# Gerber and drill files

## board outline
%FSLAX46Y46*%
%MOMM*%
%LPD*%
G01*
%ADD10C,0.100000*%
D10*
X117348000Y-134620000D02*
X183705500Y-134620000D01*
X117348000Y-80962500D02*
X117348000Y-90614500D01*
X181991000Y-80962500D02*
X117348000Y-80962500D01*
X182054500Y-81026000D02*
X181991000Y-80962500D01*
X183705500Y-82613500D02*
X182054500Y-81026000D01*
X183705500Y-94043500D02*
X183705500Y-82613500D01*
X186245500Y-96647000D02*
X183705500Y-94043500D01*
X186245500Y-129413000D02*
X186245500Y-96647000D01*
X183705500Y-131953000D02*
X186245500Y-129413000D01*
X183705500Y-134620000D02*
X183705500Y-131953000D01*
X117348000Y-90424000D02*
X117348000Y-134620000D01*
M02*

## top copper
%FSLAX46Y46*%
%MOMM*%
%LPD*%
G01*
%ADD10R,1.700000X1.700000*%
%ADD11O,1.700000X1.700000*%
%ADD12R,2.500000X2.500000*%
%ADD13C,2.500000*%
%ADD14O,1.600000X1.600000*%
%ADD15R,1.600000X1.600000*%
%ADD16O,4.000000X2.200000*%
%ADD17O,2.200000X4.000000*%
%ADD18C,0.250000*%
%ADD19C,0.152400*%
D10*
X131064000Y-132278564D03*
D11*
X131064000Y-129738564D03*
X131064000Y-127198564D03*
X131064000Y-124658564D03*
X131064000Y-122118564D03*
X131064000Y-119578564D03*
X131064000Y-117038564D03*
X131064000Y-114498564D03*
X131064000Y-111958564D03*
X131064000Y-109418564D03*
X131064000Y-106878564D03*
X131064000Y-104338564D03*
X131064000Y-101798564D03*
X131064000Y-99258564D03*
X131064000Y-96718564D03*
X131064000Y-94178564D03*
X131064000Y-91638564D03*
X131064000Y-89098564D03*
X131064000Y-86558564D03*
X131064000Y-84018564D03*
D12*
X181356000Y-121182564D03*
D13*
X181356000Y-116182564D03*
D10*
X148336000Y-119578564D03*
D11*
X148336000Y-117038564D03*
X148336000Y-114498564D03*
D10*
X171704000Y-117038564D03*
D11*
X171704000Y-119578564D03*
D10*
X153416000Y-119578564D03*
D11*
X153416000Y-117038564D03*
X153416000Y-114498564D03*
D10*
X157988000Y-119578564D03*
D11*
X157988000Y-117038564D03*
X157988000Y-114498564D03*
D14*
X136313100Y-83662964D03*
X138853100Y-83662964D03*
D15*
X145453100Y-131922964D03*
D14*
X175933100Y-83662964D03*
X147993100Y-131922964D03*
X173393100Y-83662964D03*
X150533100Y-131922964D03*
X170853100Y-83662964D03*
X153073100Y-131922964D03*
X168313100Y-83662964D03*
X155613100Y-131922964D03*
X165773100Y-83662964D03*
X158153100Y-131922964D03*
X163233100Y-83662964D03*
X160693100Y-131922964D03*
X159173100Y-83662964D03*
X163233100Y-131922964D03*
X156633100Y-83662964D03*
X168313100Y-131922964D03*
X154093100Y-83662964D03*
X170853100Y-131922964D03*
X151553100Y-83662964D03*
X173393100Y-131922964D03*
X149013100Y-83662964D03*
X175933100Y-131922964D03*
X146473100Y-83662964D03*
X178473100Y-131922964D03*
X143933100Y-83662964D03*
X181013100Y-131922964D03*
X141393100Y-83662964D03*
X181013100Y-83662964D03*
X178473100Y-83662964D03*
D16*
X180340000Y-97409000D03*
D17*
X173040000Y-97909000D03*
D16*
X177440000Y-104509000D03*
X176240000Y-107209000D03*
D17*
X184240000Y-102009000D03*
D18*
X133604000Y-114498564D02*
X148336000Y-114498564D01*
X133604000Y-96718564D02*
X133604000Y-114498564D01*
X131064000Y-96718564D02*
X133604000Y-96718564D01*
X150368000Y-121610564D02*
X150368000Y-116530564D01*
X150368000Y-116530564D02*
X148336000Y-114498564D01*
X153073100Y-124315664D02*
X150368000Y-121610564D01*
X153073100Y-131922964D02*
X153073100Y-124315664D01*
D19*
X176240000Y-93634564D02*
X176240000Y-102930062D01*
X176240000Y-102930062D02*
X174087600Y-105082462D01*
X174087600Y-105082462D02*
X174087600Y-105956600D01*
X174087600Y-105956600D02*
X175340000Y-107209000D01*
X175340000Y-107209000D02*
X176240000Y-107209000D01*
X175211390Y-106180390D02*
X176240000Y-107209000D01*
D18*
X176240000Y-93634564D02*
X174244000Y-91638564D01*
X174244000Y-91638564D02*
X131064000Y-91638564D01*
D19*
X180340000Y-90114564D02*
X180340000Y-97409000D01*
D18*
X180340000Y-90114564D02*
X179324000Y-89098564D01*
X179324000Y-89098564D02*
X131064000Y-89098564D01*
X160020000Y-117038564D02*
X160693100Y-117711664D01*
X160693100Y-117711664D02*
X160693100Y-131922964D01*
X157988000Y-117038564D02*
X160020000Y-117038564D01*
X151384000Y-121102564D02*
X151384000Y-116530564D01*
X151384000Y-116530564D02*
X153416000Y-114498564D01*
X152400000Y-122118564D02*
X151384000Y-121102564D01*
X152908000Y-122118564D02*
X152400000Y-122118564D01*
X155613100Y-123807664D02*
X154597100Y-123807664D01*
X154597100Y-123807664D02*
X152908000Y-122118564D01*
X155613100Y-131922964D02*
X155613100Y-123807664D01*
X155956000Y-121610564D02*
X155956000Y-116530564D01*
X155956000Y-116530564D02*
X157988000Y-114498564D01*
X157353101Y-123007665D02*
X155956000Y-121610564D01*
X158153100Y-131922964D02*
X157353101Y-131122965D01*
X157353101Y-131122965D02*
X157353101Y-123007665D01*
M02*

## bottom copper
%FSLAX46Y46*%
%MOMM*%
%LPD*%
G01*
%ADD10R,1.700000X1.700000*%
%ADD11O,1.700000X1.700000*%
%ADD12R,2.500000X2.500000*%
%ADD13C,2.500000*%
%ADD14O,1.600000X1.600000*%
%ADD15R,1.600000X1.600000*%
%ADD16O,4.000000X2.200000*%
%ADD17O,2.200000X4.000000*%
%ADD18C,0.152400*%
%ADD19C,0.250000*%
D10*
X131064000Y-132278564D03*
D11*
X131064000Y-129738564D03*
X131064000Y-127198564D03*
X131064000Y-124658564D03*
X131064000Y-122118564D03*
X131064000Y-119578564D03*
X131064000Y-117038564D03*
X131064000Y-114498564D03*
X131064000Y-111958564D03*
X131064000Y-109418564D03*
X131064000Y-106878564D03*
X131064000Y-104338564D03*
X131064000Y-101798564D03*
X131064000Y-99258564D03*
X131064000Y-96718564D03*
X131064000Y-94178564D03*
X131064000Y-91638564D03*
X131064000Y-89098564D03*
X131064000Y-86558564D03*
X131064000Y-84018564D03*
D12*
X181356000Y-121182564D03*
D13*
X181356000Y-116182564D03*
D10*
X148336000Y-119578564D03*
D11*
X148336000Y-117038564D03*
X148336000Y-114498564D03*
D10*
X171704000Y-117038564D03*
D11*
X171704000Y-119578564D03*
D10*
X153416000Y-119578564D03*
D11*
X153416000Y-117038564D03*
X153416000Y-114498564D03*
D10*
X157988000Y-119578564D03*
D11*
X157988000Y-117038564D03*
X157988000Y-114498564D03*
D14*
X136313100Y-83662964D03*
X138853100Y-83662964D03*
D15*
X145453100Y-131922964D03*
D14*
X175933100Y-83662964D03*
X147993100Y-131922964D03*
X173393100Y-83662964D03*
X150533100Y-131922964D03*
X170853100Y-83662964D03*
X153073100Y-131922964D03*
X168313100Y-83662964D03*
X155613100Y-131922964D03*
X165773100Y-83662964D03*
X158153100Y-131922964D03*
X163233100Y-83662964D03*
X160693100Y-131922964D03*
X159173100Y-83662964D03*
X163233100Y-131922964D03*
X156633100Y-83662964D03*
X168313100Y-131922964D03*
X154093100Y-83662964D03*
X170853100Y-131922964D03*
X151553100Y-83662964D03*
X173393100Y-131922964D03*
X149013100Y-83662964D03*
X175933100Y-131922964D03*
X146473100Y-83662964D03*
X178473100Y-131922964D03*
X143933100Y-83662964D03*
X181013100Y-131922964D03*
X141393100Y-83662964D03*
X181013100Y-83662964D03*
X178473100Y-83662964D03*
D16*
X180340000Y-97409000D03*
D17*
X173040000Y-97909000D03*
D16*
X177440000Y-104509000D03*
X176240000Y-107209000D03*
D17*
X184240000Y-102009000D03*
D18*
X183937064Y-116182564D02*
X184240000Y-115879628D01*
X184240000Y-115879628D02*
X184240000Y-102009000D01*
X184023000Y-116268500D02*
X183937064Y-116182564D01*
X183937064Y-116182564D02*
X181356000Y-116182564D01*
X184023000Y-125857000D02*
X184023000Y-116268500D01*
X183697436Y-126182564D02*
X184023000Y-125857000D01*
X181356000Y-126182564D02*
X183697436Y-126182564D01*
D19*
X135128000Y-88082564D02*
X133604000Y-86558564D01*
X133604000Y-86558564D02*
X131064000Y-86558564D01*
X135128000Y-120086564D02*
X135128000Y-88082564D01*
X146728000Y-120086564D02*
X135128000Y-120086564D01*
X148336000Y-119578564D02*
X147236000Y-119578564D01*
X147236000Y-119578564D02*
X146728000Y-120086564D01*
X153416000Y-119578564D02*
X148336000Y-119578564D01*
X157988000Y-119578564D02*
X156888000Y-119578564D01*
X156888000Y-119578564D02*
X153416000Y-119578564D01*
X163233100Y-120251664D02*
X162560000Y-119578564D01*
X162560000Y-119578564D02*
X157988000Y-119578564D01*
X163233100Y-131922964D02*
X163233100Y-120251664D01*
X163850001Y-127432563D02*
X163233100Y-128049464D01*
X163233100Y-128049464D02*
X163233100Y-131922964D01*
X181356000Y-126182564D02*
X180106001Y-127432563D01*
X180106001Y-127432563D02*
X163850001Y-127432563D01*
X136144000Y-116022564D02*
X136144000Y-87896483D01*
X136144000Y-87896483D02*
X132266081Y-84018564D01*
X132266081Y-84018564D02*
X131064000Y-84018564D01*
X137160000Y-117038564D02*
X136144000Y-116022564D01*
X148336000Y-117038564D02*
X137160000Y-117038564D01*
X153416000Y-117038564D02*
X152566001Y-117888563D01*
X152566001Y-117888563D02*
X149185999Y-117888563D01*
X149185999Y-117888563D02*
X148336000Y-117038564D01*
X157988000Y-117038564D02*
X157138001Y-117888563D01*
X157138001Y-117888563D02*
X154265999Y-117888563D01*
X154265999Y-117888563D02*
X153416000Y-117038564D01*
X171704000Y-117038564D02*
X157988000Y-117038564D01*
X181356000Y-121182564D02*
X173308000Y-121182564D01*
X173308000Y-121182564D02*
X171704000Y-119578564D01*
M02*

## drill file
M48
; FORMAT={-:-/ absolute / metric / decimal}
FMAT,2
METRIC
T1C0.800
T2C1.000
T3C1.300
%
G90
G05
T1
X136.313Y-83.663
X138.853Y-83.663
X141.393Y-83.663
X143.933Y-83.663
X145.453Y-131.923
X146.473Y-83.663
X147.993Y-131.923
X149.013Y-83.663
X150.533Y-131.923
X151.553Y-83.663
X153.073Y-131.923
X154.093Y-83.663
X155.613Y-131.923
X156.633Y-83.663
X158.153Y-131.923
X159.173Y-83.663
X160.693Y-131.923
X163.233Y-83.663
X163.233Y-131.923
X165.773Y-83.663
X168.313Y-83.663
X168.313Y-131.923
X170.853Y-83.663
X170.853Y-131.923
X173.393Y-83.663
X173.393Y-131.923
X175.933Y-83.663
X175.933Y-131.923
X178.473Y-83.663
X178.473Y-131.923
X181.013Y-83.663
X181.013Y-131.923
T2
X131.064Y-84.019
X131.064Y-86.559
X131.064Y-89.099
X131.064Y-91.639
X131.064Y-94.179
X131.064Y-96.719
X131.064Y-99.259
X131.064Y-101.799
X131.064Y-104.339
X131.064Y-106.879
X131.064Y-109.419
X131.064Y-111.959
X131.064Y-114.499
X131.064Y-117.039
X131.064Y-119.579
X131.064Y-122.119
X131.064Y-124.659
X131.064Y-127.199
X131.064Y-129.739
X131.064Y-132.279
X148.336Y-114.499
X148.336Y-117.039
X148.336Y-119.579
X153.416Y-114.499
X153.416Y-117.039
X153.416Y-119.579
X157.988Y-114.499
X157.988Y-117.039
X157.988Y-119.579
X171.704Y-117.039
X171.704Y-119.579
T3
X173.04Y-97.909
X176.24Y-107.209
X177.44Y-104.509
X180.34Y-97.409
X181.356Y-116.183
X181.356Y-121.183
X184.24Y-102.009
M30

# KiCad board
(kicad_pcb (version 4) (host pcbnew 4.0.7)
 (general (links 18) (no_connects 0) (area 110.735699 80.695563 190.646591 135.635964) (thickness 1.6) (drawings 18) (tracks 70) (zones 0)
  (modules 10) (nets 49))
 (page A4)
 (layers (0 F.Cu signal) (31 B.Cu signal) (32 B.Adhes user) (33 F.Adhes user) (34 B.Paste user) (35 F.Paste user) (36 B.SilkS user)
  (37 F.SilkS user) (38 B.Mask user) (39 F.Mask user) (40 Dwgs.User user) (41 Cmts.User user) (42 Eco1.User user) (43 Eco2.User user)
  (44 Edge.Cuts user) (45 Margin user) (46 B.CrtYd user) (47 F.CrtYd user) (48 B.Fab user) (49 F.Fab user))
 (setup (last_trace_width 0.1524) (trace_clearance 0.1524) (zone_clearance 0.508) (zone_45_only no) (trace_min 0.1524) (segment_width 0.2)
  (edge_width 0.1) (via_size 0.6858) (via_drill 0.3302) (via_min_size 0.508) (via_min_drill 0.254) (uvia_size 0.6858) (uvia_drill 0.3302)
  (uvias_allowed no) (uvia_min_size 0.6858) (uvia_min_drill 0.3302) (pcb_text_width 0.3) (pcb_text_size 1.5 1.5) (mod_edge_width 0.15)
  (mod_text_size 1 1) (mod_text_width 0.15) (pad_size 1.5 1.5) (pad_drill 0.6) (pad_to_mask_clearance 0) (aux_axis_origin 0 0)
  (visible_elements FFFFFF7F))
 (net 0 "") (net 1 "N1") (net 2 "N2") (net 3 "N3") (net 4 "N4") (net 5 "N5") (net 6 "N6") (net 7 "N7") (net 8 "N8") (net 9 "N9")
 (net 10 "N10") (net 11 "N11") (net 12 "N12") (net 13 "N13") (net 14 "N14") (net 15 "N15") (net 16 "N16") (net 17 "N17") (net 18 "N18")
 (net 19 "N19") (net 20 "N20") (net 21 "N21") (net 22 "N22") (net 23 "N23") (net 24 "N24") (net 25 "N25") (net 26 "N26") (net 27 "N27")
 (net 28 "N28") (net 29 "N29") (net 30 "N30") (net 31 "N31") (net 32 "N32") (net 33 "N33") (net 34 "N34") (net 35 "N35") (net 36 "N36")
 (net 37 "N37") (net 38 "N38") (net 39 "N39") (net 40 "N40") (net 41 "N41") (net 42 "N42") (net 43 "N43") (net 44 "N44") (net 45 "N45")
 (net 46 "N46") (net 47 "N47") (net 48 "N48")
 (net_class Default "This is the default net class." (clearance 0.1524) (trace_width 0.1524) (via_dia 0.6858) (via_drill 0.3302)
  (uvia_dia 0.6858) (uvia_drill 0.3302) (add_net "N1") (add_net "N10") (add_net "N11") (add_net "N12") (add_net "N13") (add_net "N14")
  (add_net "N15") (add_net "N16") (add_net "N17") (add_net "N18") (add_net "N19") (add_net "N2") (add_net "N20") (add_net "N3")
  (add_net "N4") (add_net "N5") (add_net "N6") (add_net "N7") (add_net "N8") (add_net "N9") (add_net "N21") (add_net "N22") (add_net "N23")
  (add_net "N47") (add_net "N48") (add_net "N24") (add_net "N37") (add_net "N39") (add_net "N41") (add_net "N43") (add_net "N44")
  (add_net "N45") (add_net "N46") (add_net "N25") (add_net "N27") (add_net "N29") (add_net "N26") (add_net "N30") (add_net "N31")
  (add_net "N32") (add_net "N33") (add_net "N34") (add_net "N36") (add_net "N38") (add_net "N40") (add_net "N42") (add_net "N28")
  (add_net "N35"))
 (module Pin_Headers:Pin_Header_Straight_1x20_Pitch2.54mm (layer B.Cu) (at 131.064 132.278564)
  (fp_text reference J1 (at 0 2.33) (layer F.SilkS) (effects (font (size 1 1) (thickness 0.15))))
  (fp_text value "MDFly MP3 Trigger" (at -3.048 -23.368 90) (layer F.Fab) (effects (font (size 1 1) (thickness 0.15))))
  (pad 1 thru_hole rect (at 0 0) (size 1.7 1.7) (drill 1) (layers *.Cu *.Mask) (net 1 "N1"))
  (pad 2 thru_hole oval (at 0 -2.54) (size 1.7 1.7) (drill 1) (layers *.Cu *.Mask) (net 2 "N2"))
  (pad 3 thru_hole oval (at 0 -5.08) (size 1.7 1.7) (drill 1) (layers *.Cu *.Mask) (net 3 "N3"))
  (pad 4 thru_hole oval (at 0 -7.62) (size 1.7 1.7) (drill 1) (layers *.Cu *.Mask) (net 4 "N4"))
  (pad 5 thru_hole oval (at 0 -10.16) (size 1.7 1.7) (drill 1) (layers *.Cu *.Mask) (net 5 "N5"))
  (pad 6 thru_hole oval (at 0 -12.7) (size 1.7 1.7) (drill 1) (layers *.Cu *.Mask) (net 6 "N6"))
  (pad 7 thru_hole oval (at 0 -15.24) (size 1.7 1.7) (drill 1) (layers *.Cu *.Mask) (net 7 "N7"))
  (pad 8 thru_hole oval (at 0 -17.78) (size 1.7 1.7) (drill 1) (layers *.Cu *.Mask) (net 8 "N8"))
  (pad 9 thru_hole oval (at 0 -20.32) (size 1.7 1.7) (drill 1) (layers *.Cu *.Mask) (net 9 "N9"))
  (pad 10 thru_hole oval (at 0 -22.86) (size 1.7 1.7) (drill 1) (layers *.Cu *.Mask) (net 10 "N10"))
  (pad 11 thru_hole oval (at 0 -25.4) (size 1.7 1.7) (drill 1) (layers *.Cu *.Mask) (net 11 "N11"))
  (pad 12 thru_hole oval (at 0 -27.94) (size 1.7 1.7) (drill 1) (layers *.Cu *.Mask) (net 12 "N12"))
  (pad 13 thru_hole oval (at 0 -30.48) (size 1.7 1.7) (drill 1) (layers *.Cu *.Mask) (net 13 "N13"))
  (pad 14 thru_hole oval (at 0 -33.02) (size 1.7 1.7) (drill 1) (layers *.Cu *.Mask) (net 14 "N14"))
  (pad 15 thru_hole oval (at 0 -35.56) (size 1.7 1.7) (drill 1) (layers *.Cu *.Mask) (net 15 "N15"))
  (pad 16 thru_hole oval (at 0 -38.1) (size 1.7 1.7) (drill 1) (layers *.Cu *.Mask) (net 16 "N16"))
  (pad 17 thru_hole oval (at 0 -40.64) (size 1.7 1.7) (drill 1) (layers *.Cu *.Mask) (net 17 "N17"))
  (pad 18 thru_hole oval (at 0 -43.18) (size 1.7 1.7) (drill 1) (layers *.Cu *.Mask) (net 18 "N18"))
  (pad 19 thru_hole oval (at 0 -45.72) (size 1.7 1.7) (drill 1) (layers *.Cu *.Mask) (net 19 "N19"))
  (pad 20 thru_hole oval (at 0 -48.26) (size 1.7 1.7) (drill 1) (layers *.Cu *.Mask) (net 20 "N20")))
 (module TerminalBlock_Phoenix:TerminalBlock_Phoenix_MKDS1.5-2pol (layer F.Cu) (at 181.356 121.182564 90)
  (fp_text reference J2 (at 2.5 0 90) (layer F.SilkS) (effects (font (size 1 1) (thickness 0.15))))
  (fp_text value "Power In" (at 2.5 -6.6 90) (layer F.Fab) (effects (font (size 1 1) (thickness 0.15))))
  (pad 1 thru_hole rect (at 0 0 90) (size 2.5 2.5) (drill 1.3) (layers *.Cu *.Mask) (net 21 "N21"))
  (pad 2 thru_hole circle (at 5 0 90) (size 2.5 2.5) (drill 1.3) (layers *.Cu *.Mask) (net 19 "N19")))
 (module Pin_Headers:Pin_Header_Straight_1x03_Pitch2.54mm (layer F.Cu) (at 148.336 119.578564 180)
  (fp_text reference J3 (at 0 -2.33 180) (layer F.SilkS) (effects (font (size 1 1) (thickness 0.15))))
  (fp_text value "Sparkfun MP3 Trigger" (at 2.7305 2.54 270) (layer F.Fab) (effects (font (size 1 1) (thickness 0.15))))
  (pad 1 thru_hole rect (at 0 0 180) (size 1.7 1.7) (drill 1) (layers *.Cu *.Mask) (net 19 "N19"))
  (pad 2 thru_hole oval (at 0 2.54 180) (size 1.7 1.7) (drill 1) (layers *.Cu *.Mask) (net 20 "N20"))
  (pad 3 thru_hole oval (at 0 5.08 180) (size 1.7 1.7) (drill 1) (layers *.Cu *.Mask) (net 15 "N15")))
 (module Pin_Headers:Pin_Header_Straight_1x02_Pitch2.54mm (layer F.Cu) (at 171.704 117.038564)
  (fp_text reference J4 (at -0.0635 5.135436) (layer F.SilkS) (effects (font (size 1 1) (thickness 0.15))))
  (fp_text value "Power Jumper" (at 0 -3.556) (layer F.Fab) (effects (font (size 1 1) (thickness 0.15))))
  (pad 1 thru_hole rect (at 0 0) (size 1.7 1.7) (drill 1) (layers *.Cu *.Mask) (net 20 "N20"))
  (pad 2 thru_hole oval (at 0 2.54) (size 1.7 1.7) (drill 1) (layers *.Cu *.Mask) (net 21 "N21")))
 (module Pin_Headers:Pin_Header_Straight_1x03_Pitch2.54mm (layer F.Cu) (at 153.416 119.578564 180)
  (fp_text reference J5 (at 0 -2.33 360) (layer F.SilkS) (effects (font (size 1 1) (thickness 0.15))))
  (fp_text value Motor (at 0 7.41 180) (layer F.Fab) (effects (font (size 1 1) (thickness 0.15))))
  (pad 1 thru_hole rect (at 0 0 180) (size 1.7 1.7) (drill 1) (layers *.Cu *.Mask) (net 19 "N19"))
  (pad 2 thru_hole oval (at 0 2.54 180) (size 1.7 1.7) (drill 1) (layers *.Cu *.Mask) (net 20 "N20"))
  (pad 3 thru_hole oval (at 0 5.08 180) (size 1.7 1.7) (drill 1) (layers *.Cu *.Mask) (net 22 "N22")))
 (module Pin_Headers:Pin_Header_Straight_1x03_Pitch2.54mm (layer F.Cu) (at 157.988 119.578564 180)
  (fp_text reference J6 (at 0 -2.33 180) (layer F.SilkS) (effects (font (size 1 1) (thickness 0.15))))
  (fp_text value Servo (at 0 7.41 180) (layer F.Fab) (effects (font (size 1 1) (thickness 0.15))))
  (pad 1 thru_hole rect (at 0 0 180) (size 1.7 1.7) (drill 1) (layers *.Cu *.Mask) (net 19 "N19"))
  (pad 2 thru_hole oval (at 0 2.54 180) (size 1.7 1.7) (drill 1) (layers *.Cu *.Mask) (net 20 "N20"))
  (pad 3 thru_hole oval (at 0 5.08 180) (size 1.7 1.7) (drill 1) (layers *.Cu *.Mask) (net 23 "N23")))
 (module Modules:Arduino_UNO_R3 (layer B.Cu) (at 145.4531 131.922964)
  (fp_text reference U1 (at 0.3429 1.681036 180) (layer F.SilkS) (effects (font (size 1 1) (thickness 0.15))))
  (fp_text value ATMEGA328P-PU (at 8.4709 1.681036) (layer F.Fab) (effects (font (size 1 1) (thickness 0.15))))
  (pad 32 thru_hole oval (at -9.14 -48.26 270) (size 1.6 1.6) (drill 0.8) (layers *.Cu *.Mask))
  (pad 31 thru_hole oval (at -6.6 -48.26 270) (size 1.6 1.6) (drill 0.8) (layers *.Cu *.Mask))
  (pad 1 thru_hole rect (at 0 0 270) (size 1.6 1.6) (drill 0.8) (layers *.Cu *.Mask) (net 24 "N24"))
  (pad 17 thru_hole oval (at 30.48 -48.26 270) (size 1.6 1.6) (drill 0.8) (layers *.Cu *.Mask) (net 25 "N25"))
  (pad 2 thru_hole oval (at 2.54 0 270) (size 1.6 1.6) (drill 0.8) (layers *.Cu *.Mask) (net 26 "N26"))
  (pad 18 thru_hole oval (at 27.94 -48.26 270) (size 1.6 1.6) (drill 0.8) (layers *.Cu *.Mask) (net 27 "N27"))
  (pad 3 thru_hole oval (at 5.08 0 270) (size 1.6 1.6) (drill 0.8) (layers *.Cu *.Mask) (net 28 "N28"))
  (pad 19 thru_hole oval (at 25.4 -48.26 270) (size 1.6 1.6) (drill 0.8) (layers *.Cu *.Mask) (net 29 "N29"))
  (pad 4 thru_hole oval (at 7.62 0 270) (size 1.6 1.6) (drill 0.8) (layers *.Cu *.Mask) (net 15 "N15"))
  (pad 20 thru_hole oval (at 22.86 -48.26 270) (size 1.6 1.6) (drill 0.8) (layers *.Cu *.Mask) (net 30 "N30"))
  (pad 5 thru_hole oval (at 10.16 0 270) (size 1.6 1.6) (drill 0.8) (layers *.Cu *.Mask) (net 22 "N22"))
  (pad 21 thru_hole oval (at 20.32 -48.26 270) (size 1.6 1.6) (drill 0.8) (layers *.Cu *.Mask) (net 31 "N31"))
  (pad 6 thru_hole oval (at 12.7 0 270) (size 1.6 1.6) (drill 0.8) (layers *.Cu *.Mask) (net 23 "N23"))
  (pad 22 thru_hole oval (at 17.78 -48.26 270) (size 1.6 1.6) (drill 0.8) (layers *.Cu *.Mask) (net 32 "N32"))
  (pad 7 thru_hole oval (at 15.24 0 270) (size 1.6 1.6) (drill 0.8) (layers *.Cu *.Mask) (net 20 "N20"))
  (pad 23 thru_hole oval (at 13.72 -48.26 270) (size 1.6 1.6) (drill 0.8) (layers *.Cu *.Mask) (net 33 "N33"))
  (pad 8 thru_hole oval (at 17.78 0 270) (size 1.6 1.6) (drill 0.8) (layers *.Cu *.Mask) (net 19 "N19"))
  (pad 24 thru_hole oval (at 11.18 -48.26 270) (size 1.6 1.6) (drill 0.8) (layers *.Cu *.Mask) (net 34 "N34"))
  (pad 9 thru_hole oval (at 22.86 0 270) (size 1.6 1.6) (drill 0.8) (layers *.Cu *.Mask) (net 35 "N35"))
  (pad 25 thru_hole oval (at 8.64 -48.26 270) (size 1.6 1.6) (drill 0.8) (layers *.Cu *.Mask) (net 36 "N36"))
  (pad 10 thru_hole oval (at 25.4 0 270) (size 1.6 1.6) (drill 0.8) (layers *.Cu *.Mask) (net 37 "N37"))
  (pad 26 thru_hole oval (at 6.1 -48.26 270) (size 1.6 1.6) (drill 0.8) (layers *.Cu *.Mask) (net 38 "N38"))
  (pad 11 thru_hole oval (at 27.94 0 270) (size 1.6 1.6) (drill 0.8) (layers *.Cu *.Mask) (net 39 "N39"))
  (pad 27 thru_hole oval (at 3.56 -48.26 270) (size 1.6 1.6) (drill 0.8) (layers *.Cu *.Mask) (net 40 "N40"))
  (pad 12 thru_hole oval (at 30.48 0 270) (size 1.6 1.6) (drill 0.8) (layers *.Cu *.Mask) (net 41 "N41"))
  (pad 28 thru_hole oval (at 1.02 -48.26 270) (size 1.6 1.6) (drill 0.8) (layers *.Cu *.Mask) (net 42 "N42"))
  (pad 13 thru_hole oval (at 33.02 0 270) (size 1.6 1.6) (drill 0.8) (layers *.Cu *.Mask) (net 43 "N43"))
  (pad 29 thru_hole oval (at -1.52 -48.26 270) (size 1.6 1.6) (drill 0.8) (layers *.Cu *.Mask))
  (pad 14 thru_hole oval (at 35.56 0 270) (size 1.6 1.6) (drill 0.8) (layers *.Cu *.Mask) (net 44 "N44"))
  (pad 30 thru_hole oval (at -4.06 -48.26 270) (size 1.6 1.6) (drill 0.8) (layers *.Cu *.Mask))
  (pad 15 thru_hole oval (at 35.56 -48.26 270) (size 1.6 1.6) (drill 0.8) (layers *.Cu *.Mask) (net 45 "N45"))
  (pad 16 thru_hole oval (at 33.02 -48.26 270) (size 1.6 1.6) (drill 0.8) (layers *.Cu *.Mask) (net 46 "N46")))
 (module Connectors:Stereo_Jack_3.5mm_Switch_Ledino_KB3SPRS (layer F.Cu) (at 180.34 97.409 180)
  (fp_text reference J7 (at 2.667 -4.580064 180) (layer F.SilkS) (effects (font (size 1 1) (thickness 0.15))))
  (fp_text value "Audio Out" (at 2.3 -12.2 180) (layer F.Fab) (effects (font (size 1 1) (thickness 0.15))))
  (pad 1 thru_hole oval (at 0 0 180) (size 4 2.2) (drill 1.3) (layers *.Cu *.Mask) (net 18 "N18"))
  (pad 4 thru_hole oval (at 7.3 -0.5 270) (size 4 2.2) (drill 1.3) (layers *.Cu *.Mask) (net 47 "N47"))
  (pad 5 thru_hole oval (at 2.9 -7.1 180) (size 4 2.2) (drill 1.3) (layers *.Cu *.Mask) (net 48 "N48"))
  (pad 2 thru_hole oval (at 4.1 -9.8 180) (size 4 2.2) (drill 1.3) (layers *.Cu *.Mask) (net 17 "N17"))
  (pad 3 thru_hole oval (at -3.9 -4.6 180) (size 2.2 4) (drill 1.3) (layers *.Cu *.Mask) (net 19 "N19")))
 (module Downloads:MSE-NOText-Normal (layer F.Cu) (at 153.924 98.242564)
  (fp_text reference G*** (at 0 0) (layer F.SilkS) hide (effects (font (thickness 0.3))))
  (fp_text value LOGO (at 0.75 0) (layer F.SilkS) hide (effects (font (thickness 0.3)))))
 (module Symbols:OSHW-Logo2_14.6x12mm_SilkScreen (layer F.Cu) (at 175.768 90.114564)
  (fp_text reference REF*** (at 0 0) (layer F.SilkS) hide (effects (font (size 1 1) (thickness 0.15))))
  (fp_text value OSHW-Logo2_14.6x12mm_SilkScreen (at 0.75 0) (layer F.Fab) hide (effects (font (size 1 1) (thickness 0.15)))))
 (gr_line (start 117.348 134.62) (end 183.7055 134.62) (layer Edge.Cuts) (width 0.1))
 (gr_line (start 117.348 80.9625) (end 117.348 90.6145) (layer Edge.Cuts) (width 0.1))
 (gr_line (start 181.991 80.9625) (end 117.348 80.9625) (layer Edge.Cuts) (width 0.1))
 (gr_line (start 182.0545 81.026) (end 181.991 80.9625) (layer Edge.Cuts) (width 0.1))
 (gr_line (start 183.7055 82.6135) (end 182.0545 81.026) (layer Edge.Cuts) (width 0.1))
 (gr_line (start 183.7055 94.0435) (end 183.7055 82.6135) (layer Edge.Cuts) (width 0.1))
 (gr_line (start 186.2455 96.647) (end 183.7055 94.0435) (layer Edge.Cuts) (width 0.1))
 (gr_line (start 186.2455 129.413) (end 186.2455 96.647) (layer Edge.Cuts) (width 0.1))
 (gr_line (start 183.7055 131.953) (end 186.2455 129.413) (layer Edge.Cuts) (width 0.1))
 (gr_line (start 183.7055 134.62) (end 183.7055 131.953) (layer Edge.Cuts) (width 0.1))
 (gr_line (start 117.348 90.424) (end 117.348 134.62) (layer Edge.Cuts) (width 0.1))
 (segment (start 133.604 114.498564) (end 148.336 114.498564) (width 0.25) (layer F.Cu) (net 15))
 (segment (start 133.604 96.718564) (end 133.604 114.498564) (width 0.25) (layer F.Cu) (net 15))
 (segment (start 131.064 96.718564) (end 133.604 96.718564) (width 0.25) (layer F.Cu) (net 15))
 (segment (start 150.368 121.610564) (end 150.368 116.530564) (width 0.25) (layer F.Cu) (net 15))
 (segment (start 150.368 116.530564) (end 148.336 114.498564) (width 0.25) (layer F.Cu) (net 15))
 (segment (start 153.0731 124.315664) (end 150.368 121.610564) (width 0.25) (layer F.Cu) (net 15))
 (segment (start 153.0731 131.922964) (end 153.0731 124.315664) (width 0.25) (layer F.Cu) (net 15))
 (segment (start 176.24 93.634564) (end 176.24 102.930062) (width 0.1524) (layer F.Cu) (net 17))
 (segment (start 176.24 102.930062) (end 174.0876 105.082462) (width 0.1524) (layer F.Cu) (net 17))
 (segment (start 174.0876 105.082462) (end 174.0876 105.9566) (width 0.1524) (layer F.Cu) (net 17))
 (segment (start 174.0876 105.9566) (end 175.34 107.209) (width 0.1524) (layer F.Cu) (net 17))
 (segment (start 175.34 107.209) (end 176.24 107.209) (width 0.1524) (layer F.Cu) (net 17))
 (segment (start 175.21139 106.18039) (end 176.24 107.209) (width 0.1524) (layer F.Cu) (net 17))
 (segment (start 176.24 93.634564) (end 174.244 91.638564) (width 0.25) (layer F.Cu) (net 17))
 (segment (start 174.244 91.638564) (end 131.064 91.638564) (width 0.25) (layer F.Cu) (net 17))
 (segment (start 180.34 90.114564) (end 180.34 97.409) (width 0.1524) (layer F.Cu) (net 18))
 (segment (start 180.34 90.114564) (end 179.324 89.098564) (width 0.25) (layer F.Cu) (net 18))
 (segment (start 179.324 89.098564) (end 131.064 89.098564) (width 0.25) (layer F.Cu) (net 18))
 (segment (start 183.937064 116.182564) (end 184.24 115.879628) (width 0.1524) (layer B.Cu) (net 19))
 (segment (start 184.24 115.879628) (end 184.24 102.009) (width 0.1524) (layer B.Cu) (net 19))
 (segment (start 184.023 116.2685) (end 183.937064 116.182564) (width 0.1524) (layer B.Cu) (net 19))
 (segment (start 183.937064 116.182564) (end 181.356 116.182564) (width 0.1524) (layer B.Cu) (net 19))
 (segment (start 184.023 125.857) (end 184.023 116.2685) (width 0.1524) (layer B.Cu) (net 19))
 (segment (start 183.697436 126.182564) (end 184.023 125.857) (width 0.1524) (layer B.Cu) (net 19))
 (segment (start 181.356 126.182564) (end 183.697436 126.182564) (width 0.1524) (layer B.Cu) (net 19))
 (segment (start 135.128 88.082564) (end 133.604 86.558564) (width 0.25) (layer B.Cu) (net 19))
 (segment (start 133.604 86.558564) (end 131.064 86.558564) (width 0.25) (layer B.Cu) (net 19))
 (segment (start 135.128 120.086564) (end 135.128 88.082564) (width 0.25) (layer B.Cu) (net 19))
 (segment (start 146.728 120.086564) (end 135.128 120.086564) (width 0.25) (layer B.Cu) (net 19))
 (segment (start 148.336 119.578564) (end 147.236 119.578564) (width 0.25) (layer B.Cu) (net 19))
 (segment (start 147.236 119.578564) (end 146.728 120.086564) (width 0.25) (layer B.Cu) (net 19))
 (segment (start 153.416 119.578564) (end 148.336 119.578564) (width 0.25) (layer B.Cu) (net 19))
 (segment (start 157.988 119.578564) (end 156.888 119.578564) (width 0.25) (layer B.Cu) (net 19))
 (segment (start 156.888 119.578564) (end 153.416 119.578564) (width 0.25) (layer B.Cu) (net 19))
 (segment (start 163.2331 120.251664) (end 162.56 119.578564) (width 0.25) (layer B.Cu) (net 19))
 (segment (start 162.56 119.578564) (end 157.988 119.578564) (width 0.25) (layer B.Cu) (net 19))
 (segment (start 163.2331 131.922964) (end 163.2331 120.251664) (width 0.25) (layer B.Cu) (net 19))
 (segment (start 163.850001 127.432563) (end 163.2331 128.049464) (width 0.25) (layer B.Cu) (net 19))
 (segment (start 163.2331 128.049464) (end 163.2331 131.922964) (width 0.25) (layer B.Cu) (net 19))
 (segment (start 181.356 126.182564) (end 180.106001 127.432563) (width 0.25) (layer B.Cu) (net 19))
 (segment (start 180.106001 127.432563) (end 163.850001 127.432563) (width 0.25) (layer B.Cu) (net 19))
 (segment (start 160.02 117.038564) (end 160.6931 117.711664) (width 0.25) (layer F.Cu) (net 20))
 (segment (start 160.6931 117.711664) (end 160.6931 131.922964) (width 0.25) (layer F.Cu) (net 20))
 (segment (start 157.988 117.038564) (end 160.02 117.038564) (width 0.25) (layer F.Cu) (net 20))
 (segment (start 136.144 116.022564) (end 136.144 87.896483) (width 0.25) (layer B.Cu) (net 20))
 (segment (start 136.144 87.896483) (end 132.266081 84.018564) (width 0.25) (layer B.Cu) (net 20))
 (segment (start 132.266081 84.018564) (end 131.064 84.018564) (width 0.25) (layer B.Cu) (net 20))
 (segment (start 137.16 117.038564) (end 136.144 116.022564) (width 0.25) (layer B.Cu) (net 20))
 (segment (start 148.336 117.038564) (end 137.16 117.038564) (width 0.25) (layer B.Cu) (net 20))
 (segment (start 153.416 117.038564) (end 152.566001 117.888563) (width 0.25) (layer B.Cu) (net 20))
 (segment (start 152.566001 117.888563) (end 149.185999 117.888563) (width 0.25) (layer B.Cu) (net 20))
 (segment (start 149.185999 117.888563) (end 148.336 117.038564) (width 0.25) (layer B.Cu) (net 20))
 (segment (start 157.988 117.038564) (end 157.138001 117.888563) (width 0.25) (layer B.Cu) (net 20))
 (segment (start 157.138001 117.888563) (end 154.265999 117.888563) (width 0.25) (layer B.Cu) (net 20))
 (segment (start 154.265999 117.888563) (end 153.416 117.038564) (width 0.25) (layer B.Cu) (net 20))
 (segment (start 171.704 117.038564) (end 157.988 117.038564) (width 0.25) (layer B.Cu) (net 20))
 (segment (start 181.356 121.182564) (end 173.308 121.182564) (width 0.25) (layer B.Cu) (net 21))
 (segment (start 173.308 121.182564) (end 171.704 119.578564) (width 0.25) (layer B.Cu) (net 21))
 (segment (start 151.384 121.102564) (end 151.384 116.530564) (width 0.25) (layer F.Cu) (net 22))
 (segment (start 151.384 116.530564) (end 153.416 114.498564) (width 0.25) (layer F.Cu) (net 22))
 (segment (start 152.4 122.118564) (end 151.384 121.102564) (width 0.25) (layer F.Cu) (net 22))
 (segment (start 152.908 122.118564) (end 152.4 122.118564) (width 0.25) (layer F.Cu) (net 22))
 (segment (start 155.6131 123.807664) (end 154.5971 123.807664) (width 0.25) (layer F.Cu) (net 22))
 (segment (start 154.5971 123.807664) (end 152.908 122.118564) (width 0.25) (layer F.Cu) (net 22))
 (segment (start 155.6131 131.922964) (end 155.6131 123.807664) (width 0.25) (layer F.Cu) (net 22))
 (segment (start 155.956 121.610564) (end 155.956 116.530564) (width 0.25) (layer F.Cu) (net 23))
 (segment (start 155.956 116.530564) (end 157.988 114.498564) (width 0.25) (layer F.Cu) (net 23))
 (segment (start 157.353101 123.007665) (end 155.956 121.610564) (width 0.25) (layer F.Cu) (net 23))
 (segment (start 158.1531 131.922964) (end 157.353101 131.122965) (width 0.25) (layer F.Cu) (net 23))
 (segment (start 157.353101 131.122965) (end 157.353101 123.007665) (width 0.25) (layer F.Cu) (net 23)))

